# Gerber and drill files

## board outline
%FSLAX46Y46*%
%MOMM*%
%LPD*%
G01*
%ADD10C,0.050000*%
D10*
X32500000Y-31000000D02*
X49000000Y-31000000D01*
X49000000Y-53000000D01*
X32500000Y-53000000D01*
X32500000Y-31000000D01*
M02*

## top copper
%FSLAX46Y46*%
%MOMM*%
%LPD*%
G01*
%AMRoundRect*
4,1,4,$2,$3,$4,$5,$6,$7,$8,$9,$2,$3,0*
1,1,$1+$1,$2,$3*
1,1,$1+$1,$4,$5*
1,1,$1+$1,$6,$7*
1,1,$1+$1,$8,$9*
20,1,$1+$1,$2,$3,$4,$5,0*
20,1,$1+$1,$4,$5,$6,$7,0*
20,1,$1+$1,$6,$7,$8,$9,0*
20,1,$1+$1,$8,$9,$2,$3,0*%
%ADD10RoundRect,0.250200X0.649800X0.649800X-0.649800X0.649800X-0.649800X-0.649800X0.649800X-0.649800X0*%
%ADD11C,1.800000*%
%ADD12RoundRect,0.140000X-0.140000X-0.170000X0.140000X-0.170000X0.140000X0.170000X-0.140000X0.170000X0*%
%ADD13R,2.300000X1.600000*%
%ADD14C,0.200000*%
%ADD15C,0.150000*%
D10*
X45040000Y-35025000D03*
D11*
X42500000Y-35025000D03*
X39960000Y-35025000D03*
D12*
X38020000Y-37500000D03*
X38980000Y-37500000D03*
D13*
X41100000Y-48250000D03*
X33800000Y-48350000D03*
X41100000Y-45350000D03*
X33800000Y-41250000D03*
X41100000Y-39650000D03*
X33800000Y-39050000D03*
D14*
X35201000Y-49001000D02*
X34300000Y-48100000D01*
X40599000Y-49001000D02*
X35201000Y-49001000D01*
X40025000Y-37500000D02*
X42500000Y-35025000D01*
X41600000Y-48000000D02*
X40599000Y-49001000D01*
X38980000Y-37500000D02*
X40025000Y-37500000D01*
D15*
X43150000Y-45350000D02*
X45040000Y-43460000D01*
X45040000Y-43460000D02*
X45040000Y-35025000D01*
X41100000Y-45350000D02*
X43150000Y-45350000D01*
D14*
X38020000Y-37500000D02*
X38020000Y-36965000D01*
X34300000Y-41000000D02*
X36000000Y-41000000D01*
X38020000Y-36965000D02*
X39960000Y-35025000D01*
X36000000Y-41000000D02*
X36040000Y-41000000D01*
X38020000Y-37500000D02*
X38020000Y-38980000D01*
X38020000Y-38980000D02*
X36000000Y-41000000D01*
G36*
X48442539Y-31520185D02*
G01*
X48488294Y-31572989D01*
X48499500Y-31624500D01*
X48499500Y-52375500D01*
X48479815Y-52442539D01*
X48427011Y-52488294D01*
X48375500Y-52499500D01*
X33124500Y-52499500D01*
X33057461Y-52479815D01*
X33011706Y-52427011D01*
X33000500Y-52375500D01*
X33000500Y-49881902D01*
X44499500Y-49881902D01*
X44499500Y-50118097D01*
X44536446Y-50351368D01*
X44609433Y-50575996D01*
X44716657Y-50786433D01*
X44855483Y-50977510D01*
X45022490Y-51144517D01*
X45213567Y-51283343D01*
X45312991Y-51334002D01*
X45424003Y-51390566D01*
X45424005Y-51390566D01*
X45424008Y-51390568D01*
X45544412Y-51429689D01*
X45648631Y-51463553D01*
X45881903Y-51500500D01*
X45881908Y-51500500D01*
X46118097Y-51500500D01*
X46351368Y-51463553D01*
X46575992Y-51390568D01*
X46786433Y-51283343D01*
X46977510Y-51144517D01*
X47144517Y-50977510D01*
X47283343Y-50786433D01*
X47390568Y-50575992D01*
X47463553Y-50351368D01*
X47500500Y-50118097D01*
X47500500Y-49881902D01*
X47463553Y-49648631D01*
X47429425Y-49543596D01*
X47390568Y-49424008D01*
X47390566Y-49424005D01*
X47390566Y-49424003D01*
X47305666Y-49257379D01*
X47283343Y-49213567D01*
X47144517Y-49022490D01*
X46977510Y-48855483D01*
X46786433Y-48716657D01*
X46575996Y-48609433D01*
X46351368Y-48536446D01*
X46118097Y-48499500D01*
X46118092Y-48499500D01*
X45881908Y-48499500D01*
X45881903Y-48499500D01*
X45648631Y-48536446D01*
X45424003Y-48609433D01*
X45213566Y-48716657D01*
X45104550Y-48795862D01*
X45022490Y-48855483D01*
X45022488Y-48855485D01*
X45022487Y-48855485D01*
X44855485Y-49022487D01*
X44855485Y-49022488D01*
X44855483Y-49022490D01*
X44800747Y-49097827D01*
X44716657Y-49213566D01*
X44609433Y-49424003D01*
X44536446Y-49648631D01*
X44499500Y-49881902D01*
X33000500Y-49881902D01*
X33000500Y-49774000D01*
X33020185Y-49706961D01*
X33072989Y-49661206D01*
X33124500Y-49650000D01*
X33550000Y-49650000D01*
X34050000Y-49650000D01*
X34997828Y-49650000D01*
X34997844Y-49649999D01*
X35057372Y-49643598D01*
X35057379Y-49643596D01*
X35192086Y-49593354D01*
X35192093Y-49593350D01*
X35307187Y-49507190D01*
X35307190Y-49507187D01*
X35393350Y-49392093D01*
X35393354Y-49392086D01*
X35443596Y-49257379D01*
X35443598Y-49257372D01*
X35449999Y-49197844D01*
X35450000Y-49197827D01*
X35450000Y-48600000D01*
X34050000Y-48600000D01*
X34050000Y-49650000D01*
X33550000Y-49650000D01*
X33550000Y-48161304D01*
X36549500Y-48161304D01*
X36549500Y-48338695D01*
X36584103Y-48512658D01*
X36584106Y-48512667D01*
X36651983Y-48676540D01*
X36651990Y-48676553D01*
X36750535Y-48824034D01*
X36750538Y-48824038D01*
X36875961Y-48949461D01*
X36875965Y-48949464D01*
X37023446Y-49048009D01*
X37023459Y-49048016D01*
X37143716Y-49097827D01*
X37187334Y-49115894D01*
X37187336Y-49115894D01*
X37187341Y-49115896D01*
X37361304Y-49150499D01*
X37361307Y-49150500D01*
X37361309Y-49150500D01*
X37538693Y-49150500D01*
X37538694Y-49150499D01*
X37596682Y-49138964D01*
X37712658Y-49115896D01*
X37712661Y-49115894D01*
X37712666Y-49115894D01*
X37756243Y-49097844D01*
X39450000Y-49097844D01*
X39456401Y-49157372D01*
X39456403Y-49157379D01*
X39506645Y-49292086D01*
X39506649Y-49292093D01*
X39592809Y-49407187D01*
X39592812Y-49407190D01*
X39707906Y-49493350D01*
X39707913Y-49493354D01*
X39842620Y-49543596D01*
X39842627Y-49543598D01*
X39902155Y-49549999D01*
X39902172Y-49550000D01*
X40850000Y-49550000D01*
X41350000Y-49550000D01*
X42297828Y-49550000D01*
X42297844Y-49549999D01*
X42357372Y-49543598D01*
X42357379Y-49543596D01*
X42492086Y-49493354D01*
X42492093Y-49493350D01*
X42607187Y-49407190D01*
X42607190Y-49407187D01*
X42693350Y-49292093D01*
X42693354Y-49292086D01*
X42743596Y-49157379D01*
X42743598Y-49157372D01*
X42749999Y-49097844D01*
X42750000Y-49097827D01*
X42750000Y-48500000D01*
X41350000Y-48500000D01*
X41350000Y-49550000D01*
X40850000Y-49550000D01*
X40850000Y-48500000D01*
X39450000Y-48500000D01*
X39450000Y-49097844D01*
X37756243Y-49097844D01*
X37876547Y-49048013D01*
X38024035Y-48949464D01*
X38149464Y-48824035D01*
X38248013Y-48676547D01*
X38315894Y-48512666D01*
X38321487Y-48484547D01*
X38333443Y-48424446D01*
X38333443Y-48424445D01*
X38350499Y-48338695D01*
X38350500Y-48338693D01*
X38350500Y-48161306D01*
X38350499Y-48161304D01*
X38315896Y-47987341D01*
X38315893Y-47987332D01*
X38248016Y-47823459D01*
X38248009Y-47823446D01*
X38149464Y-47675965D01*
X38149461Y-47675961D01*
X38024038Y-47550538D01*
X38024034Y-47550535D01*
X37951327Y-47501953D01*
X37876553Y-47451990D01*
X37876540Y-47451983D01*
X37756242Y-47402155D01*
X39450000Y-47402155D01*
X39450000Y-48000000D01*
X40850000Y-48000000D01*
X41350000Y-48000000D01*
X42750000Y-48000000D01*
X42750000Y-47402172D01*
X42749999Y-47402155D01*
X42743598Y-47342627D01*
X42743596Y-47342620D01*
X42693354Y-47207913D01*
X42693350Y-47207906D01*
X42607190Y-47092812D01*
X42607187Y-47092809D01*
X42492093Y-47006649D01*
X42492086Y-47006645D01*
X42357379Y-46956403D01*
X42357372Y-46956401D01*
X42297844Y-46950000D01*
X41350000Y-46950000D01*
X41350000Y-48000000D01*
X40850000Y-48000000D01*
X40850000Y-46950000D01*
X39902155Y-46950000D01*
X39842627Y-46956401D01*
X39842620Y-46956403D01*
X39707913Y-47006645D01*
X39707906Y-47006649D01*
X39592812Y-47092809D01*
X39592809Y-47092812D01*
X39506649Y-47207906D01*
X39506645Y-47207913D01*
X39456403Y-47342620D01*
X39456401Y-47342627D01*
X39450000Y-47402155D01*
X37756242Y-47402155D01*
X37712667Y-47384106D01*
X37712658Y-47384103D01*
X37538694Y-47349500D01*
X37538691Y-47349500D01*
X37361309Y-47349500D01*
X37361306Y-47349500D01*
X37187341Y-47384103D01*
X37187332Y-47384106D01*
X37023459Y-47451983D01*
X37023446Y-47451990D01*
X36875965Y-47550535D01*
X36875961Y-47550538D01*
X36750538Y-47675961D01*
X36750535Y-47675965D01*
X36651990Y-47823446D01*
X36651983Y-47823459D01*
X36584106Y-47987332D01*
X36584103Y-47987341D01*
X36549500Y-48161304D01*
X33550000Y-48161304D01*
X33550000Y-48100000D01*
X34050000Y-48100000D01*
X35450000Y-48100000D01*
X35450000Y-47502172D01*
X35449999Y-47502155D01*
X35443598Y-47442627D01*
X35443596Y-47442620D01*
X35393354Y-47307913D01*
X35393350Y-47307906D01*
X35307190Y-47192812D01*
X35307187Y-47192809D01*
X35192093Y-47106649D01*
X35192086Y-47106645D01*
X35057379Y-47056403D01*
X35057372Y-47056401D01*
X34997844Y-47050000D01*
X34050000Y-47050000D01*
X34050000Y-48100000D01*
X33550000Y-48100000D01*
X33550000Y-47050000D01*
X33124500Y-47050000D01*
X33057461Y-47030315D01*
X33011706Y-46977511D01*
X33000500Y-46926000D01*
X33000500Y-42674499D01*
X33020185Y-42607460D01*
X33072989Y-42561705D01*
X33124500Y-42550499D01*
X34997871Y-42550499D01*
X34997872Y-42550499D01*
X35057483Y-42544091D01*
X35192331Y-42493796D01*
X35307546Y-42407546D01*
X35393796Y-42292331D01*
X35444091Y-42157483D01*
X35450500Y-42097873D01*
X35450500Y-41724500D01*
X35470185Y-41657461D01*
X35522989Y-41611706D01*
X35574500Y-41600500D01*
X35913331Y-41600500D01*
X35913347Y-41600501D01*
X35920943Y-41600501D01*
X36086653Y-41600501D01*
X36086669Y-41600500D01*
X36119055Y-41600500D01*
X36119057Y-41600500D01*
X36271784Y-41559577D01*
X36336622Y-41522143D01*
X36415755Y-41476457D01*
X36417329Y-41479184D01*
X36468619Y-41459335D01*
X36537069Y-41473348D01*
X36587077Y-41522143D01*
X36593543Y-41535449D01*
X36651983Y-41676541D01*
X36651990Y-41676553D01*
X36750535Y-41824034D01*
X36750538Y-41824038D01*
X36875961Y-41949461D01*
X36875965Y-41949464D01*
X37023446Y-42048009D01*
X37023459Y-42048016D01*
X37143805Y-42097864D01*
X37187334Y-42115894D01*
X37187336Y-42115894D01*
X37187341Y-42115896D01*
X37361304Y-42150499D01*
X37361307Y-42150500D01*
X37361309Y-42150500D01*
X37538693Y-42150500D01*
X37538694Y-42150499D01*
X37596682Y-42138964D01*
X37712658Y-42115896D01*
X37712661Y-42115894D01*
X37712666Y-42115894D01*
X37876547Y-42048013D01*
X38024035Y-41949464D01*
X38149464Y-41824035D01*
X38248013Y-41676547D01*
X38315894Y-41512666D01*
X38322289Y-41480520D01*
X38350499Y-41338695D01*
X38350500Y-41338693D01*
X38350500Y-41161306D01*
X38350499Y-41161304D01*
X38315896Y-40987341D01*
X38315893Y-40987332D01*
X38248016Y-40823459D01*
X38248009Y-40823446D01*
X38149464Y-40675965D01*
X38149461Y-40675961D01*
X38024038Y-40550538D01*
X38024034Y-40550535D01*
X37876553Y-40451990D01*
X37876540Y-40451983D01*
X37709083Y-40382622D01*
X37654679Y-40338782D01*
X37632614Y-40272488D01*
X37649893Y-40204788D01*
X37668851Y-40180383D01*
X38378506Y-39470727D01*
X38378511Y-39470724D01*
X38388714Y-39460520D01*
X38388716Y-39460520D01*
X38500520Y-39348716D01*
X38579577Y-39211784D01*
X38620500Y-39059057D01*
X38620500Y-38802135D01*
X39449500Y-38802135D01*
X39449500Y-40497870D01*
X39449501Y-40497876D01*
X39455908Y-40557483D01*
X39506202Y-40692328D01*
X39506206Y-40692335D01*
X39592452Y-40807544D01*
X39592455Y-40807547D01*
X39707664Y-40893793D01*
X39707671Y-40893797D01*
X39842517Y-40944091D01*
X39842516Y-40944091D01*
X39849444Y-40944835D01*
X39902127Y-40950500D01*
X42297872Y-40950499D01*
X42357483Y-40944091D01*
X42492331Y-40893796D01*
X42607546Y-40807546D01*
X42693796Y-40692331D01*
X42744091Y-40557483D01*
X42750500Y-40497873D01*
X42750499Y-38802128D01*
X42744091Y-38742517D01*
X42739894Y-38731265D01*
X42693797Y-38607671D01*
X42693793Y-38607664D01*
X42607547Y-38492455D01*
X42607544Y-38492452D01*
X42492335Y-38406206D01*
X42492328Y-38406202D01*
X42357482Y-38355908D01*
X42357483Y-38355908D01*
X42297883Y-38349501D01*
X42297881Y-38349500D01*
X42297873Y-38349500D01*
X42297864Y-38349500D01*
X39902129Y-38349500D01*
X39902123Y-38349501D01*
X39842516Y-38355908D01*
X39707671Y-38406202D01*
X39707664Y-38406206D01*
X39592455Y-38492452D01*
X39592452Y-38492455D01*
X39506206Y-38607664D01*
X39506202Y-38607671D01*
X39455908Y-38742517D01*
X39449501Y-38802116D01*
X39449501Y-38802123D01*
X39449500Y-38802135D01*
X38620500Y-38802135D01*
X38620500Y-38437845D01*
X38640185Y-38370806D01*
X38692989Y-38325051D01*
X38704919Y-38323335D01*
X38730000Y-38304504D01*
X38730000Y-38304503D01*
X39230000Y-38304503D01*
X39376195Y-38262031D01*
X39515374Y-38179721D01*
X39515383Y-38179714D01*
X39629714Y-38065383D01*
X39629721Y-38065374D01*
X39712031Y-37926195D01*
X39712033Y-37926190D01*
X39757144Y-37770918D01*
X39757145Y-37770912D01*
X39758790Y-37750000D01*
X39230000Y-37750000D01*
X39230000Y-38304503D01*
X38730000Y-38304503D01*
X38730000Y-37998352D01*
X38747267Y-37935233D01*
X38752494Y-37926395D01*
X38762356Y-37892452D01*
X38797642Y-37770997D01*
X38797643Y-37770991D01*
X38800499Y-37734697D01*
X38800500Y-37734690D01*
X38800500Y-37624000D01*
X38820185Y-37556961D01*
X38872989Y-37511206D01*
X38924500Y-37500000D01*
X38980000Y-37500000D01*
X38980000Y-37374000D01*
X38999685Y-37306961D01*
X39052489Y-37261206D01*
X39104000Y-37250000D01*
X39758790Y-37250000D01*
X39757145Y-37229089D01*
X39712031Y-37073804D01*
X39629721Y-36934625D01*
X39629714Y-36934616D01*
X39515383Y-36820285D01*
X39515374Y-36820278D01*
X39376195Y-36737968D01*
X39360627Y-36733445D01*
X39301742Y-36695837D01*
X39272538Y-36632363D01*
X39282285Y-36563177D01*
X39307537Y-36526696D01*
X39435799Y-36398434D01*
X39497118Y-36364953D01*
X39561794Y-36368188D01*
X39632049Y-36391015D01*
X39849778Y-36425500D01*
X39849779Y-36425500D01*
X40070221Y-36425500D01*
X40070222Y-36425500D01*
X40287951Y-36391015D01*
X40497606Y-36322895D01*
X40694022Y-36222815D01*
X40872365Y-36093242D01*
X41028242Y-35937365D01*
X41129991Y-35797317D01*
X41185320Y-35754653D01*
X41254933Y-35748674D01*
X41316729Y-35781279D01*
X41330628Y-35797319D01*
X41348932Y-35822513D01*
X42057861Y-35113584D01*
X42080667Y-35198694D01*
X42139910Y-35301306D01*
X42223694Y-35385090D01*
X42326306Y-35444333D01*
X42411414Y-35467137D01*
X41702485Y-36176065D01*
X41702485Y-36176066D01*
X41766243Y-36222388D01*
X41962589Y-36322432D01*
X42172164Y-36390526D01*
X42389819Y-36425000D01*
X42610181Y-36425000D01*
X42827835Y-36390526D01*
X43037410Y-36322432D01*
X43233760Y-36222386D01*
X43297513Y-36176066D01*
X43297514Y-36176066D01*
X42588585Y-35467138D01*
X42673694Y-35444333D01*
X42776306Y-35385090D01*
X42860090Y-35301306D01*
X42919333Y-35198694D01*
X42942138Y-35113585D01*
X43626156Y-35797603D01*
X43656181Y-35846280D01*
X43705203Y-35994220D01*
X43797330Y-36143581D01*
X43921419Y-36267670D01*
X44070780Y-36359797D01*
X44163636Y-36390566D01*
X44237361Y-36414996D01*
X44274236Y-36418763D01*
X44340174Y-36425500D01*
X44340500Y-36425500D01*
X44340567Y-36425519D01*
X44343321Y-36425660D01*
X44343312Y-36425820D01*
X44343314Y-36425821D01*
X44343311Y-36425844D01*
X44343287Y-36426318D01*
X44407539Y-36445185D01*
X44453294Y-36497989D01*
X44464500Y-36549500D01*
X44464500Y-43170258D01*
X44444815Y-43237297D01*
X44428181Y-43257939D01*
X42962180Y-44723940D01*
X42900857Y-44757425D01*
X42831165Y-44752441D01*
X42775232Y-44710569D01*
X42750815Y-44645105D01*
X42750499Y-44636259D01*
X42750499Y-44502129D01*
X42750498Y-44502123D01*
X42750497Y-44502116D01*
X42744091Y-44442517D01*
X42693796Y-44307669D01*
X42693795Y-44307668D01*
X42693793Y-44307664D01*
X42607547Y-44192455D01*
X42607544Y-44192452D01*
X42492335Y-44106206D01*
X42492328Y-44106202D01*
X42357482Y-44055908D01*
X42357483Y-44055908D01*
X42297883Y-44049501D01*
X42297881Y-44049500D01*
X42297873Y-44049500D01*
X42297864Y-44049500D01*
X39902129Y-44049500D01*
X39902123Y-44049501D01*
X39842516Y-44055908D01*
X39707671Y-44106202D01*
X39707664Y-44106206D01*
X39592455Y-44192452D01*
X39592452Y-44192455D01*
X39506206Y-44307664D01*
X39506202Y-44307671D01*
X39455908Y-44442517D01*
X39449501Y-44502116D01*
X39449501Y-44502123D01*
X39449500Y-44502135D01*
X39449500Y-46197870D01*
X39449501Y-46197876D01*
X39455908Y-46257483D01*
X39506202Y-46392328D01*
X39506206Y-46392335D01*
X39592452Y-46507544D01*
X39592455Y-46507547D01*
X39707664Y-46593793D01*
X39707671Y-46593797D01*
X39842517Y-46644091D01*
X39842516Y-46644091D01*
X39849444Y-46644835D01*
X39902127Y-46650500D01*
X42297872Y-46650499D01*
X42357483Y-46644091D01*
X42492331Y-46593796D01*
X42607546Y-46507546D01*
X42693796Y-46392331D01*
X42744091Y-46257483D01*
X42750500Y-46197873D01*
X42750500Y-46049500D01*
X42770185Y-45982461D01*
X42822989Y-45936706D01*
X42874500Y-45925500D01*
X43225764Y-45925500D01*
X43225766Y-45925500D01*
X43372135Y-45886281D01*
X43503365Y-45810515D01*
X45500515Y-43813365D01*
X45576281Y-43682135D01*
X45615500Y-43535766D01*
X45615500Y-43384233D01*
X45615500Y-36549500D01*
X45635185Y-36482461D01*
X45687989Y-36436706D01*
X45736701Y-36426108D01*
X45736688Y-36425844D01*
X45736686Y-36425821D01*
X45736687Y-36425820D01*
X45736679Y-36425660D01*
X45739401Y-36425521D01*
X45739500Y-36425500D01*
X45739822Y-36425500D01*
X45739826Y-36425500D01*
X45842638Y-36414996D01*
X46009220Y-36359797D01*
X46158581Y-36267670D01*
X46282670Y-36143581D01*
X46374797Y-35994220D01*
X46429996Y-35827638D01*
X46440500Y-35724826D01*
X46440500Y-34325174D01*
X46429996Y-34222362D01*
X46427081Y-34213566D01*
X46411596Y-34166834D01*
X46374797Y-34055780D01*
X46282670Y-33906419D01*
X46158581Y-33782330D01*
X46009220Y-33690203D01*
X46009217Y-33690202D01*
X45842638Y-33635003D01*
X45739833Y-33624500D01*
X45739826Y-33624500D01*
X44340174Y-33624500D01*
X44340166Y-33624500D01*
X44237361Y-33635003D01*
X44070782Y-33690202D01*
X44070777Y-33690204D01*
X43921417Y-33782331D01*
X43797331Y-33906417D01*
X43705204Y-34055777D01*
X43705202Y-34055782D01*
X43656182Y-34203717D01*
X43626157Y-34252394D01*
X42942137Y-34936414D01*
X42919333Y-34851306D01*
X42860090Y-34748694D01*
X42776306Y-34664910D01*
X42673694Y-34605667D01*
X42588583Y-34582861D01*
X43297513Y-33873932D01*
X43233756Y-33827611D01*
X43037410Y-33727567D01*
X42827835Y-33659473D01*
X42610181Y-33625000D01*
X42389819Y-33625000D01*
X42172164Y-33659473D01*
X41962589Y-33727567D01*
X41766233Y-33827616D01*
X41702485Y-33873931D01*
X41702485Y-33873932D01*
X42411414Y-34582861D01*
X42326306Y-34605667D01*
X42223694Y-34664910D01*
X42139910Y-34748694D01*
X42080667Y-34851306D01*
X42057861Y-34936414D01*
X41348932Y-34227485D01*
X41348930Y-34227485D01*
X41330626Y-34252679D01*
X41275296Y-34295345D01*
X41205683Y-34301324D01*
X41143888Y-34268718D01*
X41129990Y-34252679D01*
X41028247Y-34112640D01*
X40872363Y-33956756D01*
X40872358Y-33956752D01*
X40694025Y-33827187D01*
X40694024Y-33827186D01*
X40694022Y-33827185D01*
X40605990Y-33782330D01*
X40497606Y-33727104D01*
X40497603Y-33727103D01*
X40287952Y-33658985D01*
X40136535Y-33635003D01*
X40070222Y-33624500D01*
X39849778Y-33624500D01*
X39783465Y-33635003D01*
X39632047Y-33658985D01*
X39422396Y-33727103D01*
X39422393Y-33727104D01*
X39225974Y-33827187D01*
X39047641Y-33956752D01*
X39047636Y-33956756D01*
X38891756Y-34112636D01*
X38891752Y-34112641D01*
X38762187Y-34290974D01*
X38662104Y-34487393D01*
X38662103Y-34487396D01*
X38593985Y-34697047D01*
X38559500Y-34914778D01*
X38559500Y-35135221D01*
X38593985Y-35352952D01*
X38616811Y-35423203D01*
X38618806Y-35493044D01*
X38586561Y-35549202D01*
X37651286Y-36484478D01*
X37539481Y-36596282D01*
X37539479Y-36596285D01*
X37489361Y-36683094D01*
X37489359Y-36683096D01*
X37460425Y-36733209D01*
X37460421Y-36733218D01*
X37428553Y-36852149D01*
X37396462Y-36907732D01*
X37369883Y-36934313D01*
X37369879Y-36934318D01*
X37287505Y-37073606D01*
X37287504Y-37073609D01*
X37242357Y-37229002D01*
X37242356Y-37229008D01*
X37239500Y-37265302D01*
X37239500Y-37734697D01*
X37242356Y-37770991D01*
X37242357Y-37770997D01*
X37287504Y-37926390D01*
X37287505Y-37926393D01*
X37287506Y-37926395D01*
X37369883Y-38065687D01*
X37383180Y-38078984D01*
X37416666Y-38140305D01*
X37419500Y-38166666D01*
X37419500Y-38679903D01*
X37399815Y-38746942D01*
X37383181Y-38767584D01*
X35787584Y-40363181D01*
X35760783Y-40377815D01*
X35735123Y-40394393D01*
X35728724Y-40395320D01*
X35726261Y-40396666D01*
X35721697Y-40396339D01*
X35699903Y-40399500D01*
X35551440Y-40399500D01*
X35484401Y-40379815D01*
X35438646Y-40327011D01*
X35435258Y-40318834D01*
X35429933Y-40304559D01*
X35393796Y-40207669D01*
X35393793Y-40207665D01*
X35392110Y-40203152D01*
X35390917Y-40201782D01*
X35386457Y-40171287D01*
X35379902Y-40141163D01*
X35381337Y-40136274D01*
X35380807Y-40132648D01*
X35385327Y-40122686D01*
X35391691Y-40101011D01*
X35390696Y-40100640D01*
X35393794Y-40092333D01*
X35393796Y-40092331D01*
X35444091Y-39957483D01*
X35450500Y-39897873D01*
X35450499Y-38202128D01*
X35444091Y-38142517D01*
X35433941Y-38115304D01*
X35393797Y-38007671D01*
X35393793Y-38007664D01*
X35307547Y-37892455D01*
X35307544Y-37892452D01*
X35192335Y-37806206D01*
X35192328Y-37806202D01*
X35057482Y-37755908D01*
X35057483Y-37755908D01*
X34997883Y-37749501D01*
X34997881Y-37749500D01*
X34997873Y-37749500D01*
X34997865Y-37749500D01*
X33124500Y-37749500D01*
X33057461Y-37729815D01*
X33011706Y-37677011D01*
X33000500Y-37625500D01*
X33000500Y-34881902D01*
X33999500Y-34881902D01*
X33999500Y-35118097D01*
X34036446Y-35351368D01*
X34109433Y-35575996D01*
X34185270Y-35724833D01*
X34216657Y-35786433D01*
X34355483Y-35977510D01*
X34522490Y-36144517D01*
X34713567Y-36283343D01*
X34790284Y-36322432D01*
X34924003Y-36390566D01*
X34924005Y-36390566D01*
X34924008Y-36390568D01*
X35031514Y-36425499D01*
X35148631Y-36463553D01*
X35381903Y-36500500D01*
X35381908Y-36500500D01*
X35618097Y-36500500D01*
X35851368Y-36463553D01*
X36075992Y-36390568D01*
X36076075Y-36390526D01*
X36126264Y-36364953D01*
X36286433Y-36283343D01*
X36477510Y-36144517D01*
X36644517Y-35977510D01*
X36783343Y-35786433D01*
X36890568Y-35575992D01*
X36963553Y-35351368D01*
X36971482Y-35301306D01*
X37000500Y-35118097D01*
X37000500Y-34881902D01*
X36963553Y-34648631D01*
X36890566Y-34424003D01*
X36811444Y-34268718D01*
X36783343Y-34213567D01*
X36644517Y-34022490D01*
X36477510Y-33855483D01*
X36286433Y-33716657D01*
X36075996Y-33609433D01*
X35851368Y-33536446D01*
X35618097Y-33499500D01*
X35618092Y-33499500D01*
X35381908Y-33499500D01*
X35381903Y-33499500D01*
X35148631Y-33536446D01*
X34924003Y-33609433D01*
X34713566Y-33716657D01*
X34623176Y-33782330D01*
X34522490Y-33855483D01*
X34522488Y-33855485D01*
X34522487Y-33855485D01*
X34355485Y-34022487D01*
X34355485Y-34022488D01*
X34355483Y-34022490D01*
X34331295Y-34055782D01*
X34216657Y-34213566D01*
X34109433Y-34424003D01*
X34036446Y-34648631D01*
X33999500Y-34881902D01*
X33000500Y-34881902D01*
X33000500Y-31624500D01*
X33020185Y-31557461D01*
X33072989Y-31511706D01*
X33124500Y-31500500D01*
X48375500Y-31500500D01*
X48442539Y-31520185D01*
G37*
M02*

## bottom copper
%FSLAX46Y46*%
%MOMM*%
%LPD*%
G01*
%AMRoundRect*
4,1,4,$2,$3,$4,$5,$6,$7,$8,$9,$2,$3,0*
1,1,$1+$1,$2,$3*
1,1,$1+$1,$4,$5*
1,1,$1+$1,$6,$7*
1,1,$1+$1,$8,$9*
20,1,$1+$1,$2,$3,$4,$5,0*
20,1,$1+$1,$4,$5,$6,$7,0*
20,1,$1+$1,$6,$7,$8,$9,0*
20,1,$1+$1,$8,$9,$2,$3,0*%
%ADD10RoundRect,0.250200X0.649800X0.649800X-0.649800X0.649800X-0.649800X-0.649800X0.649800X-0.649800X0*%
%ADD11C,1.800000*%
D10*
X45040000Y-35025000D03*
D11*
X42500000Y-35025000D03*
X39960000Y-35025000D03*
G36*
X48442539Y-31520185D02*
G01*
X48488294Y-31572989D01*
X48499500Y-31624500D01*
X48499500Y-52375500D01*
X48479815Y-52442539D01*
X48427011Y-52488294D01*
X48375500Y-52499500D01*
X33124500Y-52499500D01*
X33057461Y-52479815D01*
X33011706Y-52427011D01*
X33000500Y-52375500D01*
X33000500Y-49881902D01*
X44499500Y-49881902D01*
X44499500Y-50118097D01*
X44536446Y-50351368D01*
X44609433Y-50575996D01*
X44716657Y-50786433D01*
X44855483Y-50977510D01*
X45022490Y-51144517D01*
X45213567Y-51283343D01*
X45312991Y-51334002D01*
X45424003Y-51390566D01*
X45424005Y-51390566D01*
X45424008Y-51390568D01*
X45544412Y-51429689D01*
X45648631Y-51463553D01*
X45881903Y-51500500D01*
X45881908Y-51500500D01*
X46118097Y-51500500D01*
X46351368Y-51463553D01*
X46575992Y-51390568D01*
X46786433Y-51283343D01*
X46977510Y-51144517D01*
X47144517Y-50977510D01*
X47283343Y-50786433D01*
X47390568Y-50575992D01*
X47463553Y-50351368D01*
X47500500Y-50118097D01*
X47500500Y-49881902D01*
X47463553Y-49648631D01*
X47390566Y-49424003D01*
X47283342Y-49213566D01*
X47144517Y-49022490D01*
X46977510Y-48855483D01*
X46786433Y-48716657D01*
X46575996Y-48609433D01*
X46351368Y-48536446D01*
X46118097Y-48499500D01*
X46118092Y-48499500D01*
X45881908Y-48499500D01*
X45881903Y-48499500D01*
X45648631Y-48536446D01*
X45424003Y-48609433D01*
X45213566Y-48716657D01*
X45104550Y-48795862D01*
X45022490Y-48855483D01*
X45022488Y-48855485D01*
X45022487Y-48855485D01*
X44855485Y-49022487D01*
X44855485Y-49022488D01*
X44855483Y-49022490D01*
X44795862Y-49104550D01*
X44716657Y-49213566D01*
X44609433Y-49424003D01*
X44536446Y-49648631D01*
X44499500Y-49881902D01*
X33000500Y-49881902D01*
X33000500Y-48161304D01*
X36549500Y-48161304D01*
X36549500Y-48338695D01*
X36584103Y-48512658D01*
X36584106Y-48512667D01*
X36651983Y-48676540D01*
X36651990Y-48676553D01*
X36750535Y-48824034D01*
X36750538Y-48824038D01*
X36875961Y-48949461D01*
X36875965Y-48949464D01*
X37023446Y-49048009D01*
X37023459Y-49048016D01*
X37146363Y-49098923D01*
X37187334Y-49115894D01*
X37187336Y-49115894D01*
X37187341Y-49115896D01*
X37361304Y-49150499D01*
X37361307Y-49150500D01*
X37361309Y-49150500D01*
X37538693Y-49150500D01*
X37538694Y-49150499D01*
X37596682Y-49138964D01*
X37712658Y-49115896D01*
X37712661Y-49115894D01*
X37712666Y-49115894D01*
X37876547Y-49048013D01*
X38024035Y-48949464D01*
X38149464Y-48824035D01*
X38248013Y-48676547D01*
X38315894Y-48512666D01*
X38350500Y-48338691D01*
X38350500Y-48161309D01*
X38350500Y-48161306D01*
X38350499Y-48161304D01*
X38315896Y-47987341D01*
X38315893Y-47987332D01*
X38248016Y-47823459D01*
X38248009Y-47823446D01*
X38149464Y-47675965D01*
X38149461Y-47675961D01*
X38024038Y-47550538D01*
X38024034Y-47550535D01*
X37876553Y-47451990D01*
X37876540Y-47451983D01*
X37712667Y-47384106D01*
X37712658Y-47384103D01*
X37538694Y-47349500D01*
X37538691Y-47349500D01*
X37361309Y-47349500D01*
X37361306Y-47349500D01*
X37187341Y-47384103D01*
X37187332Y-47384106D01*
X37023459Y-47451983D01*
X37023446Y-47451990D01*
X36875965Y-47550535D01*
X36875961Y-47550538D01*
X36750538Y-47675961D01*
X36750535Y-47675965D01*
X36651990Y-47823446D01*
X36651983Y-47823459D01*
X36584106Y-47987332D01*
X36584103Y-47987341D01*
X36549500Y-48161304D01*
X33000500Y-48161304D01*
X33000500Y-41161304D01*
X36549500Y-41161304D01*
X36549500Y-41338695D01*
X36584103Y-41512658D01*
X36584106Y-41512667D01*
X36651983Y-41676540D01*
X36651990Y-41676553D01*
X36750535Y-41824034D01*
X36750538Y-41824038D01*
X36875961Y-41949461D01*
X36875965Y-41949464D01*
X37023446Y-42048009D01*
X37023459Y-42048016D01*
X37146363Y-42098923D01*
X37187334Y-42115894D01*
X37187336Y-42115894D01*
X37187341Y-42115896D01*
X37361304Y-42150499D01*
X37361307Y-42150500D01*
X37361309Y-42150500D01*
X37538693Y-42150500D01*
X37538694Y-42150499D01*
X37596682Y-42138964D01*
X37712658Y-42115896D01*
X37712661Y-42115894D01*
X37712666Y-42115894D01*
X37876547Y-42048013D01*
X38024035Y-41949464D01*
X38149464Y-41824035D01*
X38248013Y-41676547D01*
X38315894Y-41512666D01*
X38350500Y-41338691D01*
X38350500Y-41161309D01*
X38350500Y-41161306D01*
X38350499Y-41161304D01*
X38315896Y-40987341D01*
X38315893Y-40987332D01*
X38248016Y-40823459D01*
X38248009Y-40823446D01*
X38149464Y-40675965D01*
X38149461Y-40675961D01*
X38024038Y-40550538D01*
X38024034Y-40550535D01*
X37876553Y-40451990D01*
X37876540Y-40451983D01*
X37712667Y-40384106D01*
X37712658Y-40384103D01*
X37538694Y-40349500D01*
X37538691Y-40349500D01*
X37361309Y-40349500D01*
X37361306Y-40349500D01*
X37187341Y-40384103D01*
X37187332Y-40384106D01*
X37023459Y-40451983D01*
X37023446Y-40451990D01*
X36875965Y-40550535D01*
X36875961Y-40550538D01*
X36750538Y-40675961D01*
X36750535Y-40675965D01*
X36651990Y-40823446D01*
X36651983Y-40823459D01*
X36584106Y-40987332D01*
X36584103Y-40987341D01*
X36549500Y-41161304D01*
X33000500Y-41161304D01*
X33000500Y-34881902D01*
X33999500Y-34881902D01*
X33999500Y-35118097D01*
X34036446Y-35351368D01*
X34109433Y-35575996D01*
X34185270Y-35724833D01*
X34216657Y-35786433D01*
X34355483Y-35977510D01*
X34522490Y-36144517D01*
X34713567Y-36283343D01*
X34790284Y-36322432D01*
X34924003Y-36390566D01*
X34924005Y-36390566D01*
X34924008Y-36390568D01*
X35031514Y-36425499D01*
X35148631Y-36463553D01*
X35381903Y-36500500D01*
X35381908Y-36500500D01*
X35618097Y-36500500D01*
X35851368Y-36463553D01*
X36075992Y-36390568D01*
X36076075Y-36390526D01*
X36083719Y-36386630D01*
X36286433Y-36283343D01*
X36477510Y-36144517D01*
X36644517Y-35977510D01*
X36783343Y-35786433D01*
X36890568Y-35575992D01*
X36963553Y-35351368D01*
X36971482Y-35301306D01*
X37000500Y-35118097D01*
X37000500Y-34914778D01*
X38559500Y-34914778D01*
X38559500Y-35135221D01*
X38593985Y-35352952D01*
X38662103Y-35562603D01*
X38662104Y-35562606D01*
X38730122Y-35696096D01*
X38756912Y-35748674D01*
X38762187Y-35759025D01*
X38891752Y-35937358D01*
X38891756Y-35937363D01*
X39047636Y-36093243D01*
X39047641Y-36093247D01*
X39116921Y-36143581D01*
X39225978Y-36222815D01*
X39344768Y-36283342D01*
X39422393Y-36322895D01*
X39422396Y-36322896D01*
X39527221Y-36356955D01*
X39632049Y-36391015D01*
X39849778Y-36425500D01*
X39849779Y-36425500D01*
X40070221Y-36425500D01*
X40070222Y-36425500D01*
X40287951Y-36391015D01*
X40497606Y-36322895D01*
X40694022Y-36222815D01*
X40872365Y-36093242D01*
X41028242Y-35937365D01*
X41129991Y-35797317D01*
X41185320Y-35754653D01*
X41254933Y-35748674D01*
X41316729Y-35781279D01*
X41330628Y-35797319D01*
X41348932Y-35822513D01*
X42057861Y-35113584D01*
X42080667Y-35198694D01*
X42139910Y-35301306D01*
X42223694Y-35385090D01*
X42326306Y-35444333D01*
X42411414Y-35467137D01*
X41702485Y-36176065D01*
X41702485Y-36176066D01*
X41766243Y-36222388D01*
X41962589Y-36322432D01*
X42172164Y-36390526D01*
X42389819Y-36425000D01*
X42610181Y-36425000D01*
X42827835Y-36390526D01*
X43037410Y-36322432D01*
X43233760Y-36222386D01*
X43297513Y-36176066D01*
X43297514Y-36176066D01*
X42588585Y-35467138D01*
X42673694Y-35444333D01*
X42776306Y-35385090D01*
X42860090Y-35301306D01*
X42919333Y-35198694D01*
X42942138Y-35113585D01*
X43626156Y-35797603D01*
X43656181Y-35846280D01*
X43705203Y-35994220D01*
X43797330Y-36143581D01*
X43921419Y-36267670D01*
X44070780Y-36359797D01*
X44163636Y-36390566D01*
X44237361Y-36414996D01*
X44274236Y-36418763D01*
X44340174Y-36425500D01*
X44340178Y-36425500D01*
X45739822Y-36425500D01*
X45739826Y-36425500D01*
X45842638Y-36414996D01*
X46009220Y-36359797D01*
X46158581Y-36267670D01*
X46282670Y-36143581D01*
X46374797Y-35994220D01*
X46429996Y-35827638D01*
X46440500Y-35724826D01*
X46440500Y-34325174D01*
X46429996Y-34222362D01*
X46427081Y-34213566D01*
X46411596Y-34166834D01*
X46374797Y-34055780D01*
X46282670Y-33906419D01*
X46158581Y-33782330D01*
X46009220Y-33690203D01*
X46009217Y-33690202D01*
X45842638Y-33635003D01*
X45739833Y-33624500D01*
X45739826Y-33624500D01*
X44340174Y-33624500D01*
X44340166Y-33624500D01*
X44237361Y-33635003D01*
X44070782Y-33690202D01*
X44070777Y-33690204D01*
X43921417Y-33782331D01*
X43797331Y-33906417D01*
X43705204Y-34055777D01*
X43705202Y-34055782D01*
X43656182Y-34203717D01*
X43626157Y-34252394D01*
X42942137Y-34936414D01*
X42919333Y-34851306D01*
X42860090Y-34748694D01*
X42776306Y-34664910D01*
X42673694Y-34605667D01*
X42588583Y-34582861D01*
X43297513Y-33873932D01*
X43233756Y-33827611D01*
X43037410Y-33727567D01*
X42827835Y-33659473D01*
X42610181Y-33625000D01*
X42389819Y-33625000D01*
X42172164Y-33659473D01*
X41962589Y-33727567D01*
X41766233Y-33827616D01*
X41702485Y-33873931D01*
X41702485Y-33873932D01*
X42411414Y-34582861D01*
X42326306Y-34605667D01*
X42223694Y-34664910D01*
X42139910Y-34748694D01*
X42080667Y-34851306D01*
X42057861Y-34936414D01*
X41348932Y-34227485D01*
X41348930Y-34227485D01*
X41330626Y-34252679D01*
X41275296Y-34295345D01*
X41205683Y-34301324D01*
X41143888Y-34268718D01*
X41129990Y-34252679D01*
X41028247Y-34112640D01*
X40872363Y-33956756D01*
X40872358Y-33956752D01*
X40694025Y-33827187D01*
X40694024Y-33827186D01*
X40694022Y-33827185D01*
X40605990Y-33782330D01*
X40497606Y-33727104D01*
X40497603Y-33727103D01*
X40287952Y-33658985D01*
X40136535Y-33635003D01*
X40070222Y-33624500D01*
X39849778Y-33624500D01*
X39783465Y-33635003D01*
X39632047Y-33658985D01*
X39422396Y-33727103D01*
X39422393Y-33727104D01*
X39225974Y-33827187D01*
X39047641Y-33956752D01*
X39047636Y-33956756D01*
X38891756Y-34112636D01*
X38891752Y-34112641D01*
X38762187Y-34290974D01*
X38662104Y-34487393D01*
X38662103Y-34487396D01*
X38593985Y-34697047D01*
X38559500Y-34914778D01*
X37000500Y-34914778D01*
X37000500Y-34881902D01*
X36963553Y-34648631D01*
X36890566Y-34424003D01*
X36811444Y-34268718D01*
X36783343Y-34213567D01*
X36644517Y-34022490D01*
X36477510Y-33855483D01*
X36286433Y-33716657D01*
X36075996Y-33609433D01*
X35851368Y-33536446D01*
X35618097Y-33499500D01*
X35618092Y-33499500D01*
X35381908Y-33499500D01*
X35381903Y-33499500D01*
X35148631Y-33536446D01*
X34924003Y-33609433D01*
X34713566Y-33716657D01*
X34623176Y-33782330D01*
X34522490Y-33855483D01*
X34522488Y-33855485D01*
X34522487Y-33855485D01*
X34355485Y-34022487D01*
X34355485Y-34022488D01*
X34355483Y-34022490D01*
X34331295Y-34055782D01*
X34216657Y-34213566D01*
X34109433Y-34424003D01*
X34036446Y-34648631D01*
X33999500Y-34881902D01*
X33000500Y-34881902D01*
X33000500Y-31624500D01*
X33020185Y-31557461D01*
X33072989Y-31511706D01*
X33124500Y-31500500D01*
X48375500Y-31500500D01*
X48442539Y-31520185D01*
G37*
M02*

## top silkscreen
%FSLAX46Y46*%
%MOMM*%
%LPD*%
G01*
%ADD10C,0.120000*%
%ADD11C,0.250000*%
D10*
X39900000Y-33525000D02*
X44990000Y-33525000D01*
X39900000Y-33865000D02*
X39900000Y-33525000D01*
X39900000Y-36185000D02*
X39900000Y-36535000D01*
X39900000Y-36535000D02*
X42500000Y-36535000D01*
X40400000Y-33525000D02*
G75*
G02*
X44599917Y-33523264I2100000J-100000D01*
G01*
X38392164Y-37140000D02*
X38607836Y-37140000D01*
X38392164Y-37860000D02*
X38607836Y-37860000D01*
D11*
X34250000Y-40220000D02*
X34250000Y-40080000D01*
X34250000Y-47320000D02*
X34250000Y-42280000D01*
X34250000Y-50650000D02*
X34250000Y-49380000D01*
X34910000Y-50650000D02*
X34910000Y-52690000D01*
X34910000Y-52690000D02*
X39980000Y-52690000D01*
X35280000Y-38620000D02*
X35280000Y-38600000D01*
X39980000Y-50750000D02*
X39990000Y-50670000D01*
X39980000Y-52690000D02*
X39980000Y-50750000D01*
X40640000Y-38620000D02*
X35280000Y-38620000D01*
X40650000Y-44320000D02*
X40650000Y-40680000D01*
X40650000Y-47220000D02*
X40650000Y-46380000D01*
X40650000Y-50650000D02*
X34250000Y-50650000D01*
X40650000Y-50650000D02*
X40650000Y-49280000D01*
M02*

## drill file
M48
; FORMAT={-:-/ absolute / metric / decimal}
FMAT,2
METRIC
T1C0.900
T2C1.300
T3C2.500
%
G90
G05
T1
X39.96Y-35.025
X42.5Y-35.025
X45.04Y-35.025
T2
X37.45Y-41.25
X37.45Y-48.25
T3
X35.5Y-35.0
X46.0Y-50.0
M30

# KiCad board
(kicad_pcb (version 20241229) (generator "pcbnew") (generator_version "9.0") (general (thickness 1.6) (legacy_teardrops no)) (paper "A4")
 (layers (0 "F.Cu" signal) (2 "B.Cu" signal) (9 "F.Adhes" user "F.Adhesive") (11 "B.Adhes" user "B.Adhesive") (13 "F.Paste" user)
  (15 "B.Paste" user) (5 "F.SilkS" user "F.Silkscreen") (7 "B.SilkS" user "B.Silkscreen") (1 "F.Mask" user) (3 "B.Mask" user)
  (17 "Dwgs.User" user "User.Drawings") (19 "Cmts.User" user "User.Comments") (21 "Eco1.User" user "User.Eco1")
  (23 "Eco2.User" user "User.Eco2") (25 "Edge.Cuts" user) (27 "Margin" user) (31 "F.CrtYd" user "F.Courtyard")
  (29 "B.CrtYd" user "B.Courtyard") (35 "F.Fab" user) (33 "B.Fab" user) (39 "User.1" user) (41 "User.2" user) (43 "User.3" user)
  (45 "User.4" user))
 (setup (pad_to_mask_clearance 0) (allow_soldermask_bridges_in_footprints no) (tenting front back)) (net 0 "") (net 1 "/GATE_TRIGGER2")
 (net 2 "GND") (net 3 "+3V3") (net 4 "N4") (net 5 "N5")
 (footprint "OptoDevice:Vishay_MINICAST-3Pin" (layer "F.Cu") (at 45.04 35.025 180)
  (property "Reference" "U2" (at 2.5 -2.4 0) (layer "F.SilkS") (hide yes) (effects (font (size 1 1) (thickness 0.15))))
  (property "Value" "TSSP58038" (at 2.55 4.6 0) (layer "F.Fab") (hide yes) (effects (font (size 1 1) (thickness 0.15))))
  (fp_line (start 5.14 1.5) (end 0.05 1.5) (stroke (width 0.12) (type solid)) (layer "F.SilkS"))
  (fp_line (start 5.14 1.16) (end 5.14 1.5) (stroke (width 0.12) (type solid)) (layer "F.SilkS"))
  (fp_line (start 5.14 -1.16) (end 5.14 -1.51) (stroke (width 0.12) (type solid)) (layer "F.SilkS"))
  (fp_line (start 5.14 -1.51) (end 2.54 -1.51) (stroke (width 0.12) (type solid)) (layer "F.SilkS"))
  (fp_arc (start 4.64 1.5) (mid 2.540869 3.502379) (end 0.440083 1.501736) (stroke (width 0.12) (type solid)) (layer "F.SilkS"))
  (pad "1" thru_hole roundrect (at 0 0 180) (size 1.8 1.8) (drill 0.9) (layers "*.Cu" "*.Mask") (remove_unused_layers no)
   (roundrect_rratio 0.139) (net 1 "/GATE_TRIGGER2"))
  (pad "2" thru_hole circle (at 2.54 0 180) (size 1.8 1.8) (drill 0.9) (layers "*.Cu" "*.Mask") (remove_unused_layers no) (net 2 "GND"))
  (pad "3" thru_hole circle (at 5.08 0 180) (size 1.8 1.8) (drill 0.9) (layers "*.Cu" "*.Mask") (remove_unused_layers no) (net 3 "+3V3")))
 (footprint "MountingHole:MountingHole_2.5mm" (layer "F.Cu") (at 35.5 35)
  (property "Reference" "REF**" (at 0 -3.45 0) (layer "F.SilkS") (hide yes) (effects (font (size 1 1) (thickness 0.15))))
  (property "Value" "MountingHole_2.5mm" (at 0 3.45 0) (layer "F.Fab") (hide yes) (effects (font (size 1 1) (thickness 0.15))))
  (pad "" np_thru_hole circle (at 0 0) (size 2.5 2.5) (drill 2.5) (layers "*.Cu" "*.Mask")))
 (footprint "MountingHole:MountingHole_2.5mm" (layer "F.Cu") (at 46 50)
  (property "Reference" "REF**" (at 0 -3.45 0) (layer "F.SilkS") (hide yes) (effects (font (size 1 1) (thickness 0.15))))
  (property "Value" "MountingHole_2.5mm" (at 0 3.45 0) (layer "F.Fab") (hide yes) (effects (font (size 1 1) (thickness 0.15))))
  (pad "" np_thru_hole circle (at 0 0) (size 2.5 2.5) (drill 2.5) (layers "*.Cu" "*.Mask")))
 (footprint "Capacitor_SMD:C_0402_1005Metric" (layer "F.Cu") (at 38.5 37.5)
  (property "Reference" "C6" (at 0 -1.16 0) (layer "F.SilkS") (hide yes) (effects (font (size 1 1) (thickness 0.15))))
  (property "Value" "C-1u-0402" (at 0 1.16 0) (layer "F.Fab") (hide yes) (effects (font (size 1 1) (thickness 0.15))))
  (fp_line (start -0.107836 -0.36) (end 0.107836 -0.36) (stroke (width 0.12) (type solid)) (layer "F.SilkS"))
  (fp_line (start -0.107836 0.36) (end 0.107836 0.36) (stroke (width 0.12) (type solid)) (layer "F.SilkS"))
  (pad "1" smd roundrect (at -0.48 0) (size 0.56 0.62) (layers "F.Cu" "F.Mask" "F.Paste") (roundrect_rratio 0.25) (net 3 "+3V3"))
  (pad "2" smd roundrect (at 0.48 0) (size 0.56 0.62) (layers "F.Cu" "F.Mask" "F.Paste") (roundrect_rratio 0.25) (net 2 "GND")))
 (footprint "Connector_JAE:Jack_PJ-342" (layer "F.Cu") (at 37.5 45 180)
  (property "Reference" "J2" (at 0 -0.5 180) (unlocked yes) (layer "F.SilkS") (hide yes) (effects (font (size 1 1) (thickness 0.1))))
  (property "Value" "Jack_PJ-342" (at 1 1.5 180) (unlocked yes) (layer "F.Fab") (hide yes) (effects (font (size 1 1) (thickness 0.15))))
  (fp_line (start 3.25 4.78) (end 3.25 4.92) (stroke (width 0.25) (type solid)) (layer "F.SilkS"))
  (fp_line (start 3.25 -2.32) (end 3.25 2.72) (stroke (width 0.25) (type solid)) (layer "F.SilkS"))
  (fp_line (start 3.25 -5.65) (end 3.25 -4.38) (stroke (width 0.25) (type solid)) (layer "F.SilkS"))
  (fp_line (start 2.59 -5.65) (end 2.59 -7.69) (stroke (width 0.25) (type solid)) (layer "F.SilkS"))
  (fp_line (start 2.59 -7.69) (end -2.48 -7.69) (stroke (width 0.25) (type solid)) (layer "F.SilkS"))
  (fp_line (start 2.22 6.38) (end 2.22 6.4) (stroke (width 0.25) (type solid)) (layer "F.SilkS"))
  (fp_line (start -2.48 -5.75) (end -2.49 -5.67) (stroke (width 0.25) (type solid)) (layer "F.SilkS"))
  (fp_line (start -2.48 -7.69) (end -2.48 -5.75) (stroke (width 0.25) (type solid)) (layer "F.SilkS"))
  (fp_line (start -3.14 6.38) (end 2.22 6.38) (stroke (width 0.25) (type solid)) (layer "F.SilkS"))
  (fp_line (start -3.15 0.68) (end -3.15 4.32) (stroke (width 0.25) (type solid)) (layer "F.SilkS"))
  (fp_line (start -3.15 -2.22) (end -3.15 -1.38) (stroke (width 0.25) (type solid)) (layer "F.SilkS"))
  (fp_line (start -3.15 -5.65) (end 3.25 -5.65) (stroke (width 0.25) (type solid)) (layer "F.SilkS"))
  (fp_line (start -3.15 -5.65) (end -3.15 -4.28) (stroke (width 0.25) (type solid)) (layer "F.SilkS"))
  (pad "" np_thru_hole circle (at 0.05 -3.25 180) (size 1.3 1.3) (drill 1.3) (layers "*.Cu" "*.Mask"))
  (pad "" np_thru_hole circle (at 0.05 3.75 180) (size 1.3 1.3) (drill 1.3) (layers "*.Cu" "*.Mask"))
  (pad "2" smd rect (at -3.6 -3.25 180) (size 2.3 1.6) (layers "F.Cu" "F.Mask" "F.Paste") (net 2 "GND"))
  (pad "3" smd rect (at 3.7 -3.35 180) (size 2.3 1.6) (layers "F.Cu" "F.Mask" "F.Paste") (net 2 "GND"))
  (pad "4" smd rect (at -3.6 -0.35 180) (size 2.3 1.6) (layers "F.Cu" "F.Mask" "F.Paste") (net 1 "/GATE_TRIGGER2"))
  (pad "5" smd rect (at 3.7 3.75 180) (size 2.3 1.6) (layers "F.Cu" "F.Mask" "F.Paste") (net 3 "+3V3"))
  (pad "6" smd rect (at -3.6 5.35 180) (size 2.3 1.6) (layers "F.Cu" "F.Mask" "F.Paste") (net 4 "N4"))
  (pad "7" smd rect (at 3.7 5.95 180) (size 2.3 1.6) (layers "F.Cu" "F.Mask" "F.Paste") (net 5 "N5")))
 (gr_rect (start 32.5 31) (end 49 53) (stroke (width 0.05) (type solid)) (fill no) (layer "Edge.Cuts"))
 (segment (start 35.201 49.001) (end 34.3 48.1) (width 0.2) (layer "F.Cu") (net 2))
 (segment (start 40.599 49.001) (end 35.201 49.001) (width 0.2) (layer "F.Cu") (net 2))
 (segment (start 40.025 37.5) (end 42.5 35.025) (width 0.2) (layer "F.Cu") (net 2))
 (segment (start 41.6 48) (end 40.599 49.001) (width 0.2) (layer "F.Cu") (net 2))
 (segment (start 38.98 37.5) (end 40.025 37.5) (width 0.2) (layer "F.Cu") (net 2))
 (segment (start 43.15 45.35) (end 45.04 43.46) (width 0.15) (layer "F.Cu") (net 1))
 (segment (start 45.04 43.46) (end 45.04 35.025) (width 0.15) (layer "F.Cu") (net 1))
 (segment (start 41.1 45.35) (end 43.15 45.35) (width 0.15) (layer "F.Cu") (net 1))
 (segment (start 38.02 37.5) (end 38.02 36.965) (width 0.2) (layer "F.Cu") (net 3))
 (segment (start 34.3 41) (end 36 41) (width 0.2) (layer "F.Cu") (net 3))
 (segment (start 38.02 36.965) (end 39.96 35.025) (width 0.2) (layer "F.Cu") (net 3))
 (segment (start 36 41) (end 36.04 41) (width 0.2) (layer "F.Cu") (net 3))
 (segment (start 38.02 37.5) (end 38.02 38.98) (width 0.2) (layer "F.Cu") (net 3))
 (segment (start 38.02 38.98) (end 36 41) (width 0.2) (layer "F.Cu") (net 3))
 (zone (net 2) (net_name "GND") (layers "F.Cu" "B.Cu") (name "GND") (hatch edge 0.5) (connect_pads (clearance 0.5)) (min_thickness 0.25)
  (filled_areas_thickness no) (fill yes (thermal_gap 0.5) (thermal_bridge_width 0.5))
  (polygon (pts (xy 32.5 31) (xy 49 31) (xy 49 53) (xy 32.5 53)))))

